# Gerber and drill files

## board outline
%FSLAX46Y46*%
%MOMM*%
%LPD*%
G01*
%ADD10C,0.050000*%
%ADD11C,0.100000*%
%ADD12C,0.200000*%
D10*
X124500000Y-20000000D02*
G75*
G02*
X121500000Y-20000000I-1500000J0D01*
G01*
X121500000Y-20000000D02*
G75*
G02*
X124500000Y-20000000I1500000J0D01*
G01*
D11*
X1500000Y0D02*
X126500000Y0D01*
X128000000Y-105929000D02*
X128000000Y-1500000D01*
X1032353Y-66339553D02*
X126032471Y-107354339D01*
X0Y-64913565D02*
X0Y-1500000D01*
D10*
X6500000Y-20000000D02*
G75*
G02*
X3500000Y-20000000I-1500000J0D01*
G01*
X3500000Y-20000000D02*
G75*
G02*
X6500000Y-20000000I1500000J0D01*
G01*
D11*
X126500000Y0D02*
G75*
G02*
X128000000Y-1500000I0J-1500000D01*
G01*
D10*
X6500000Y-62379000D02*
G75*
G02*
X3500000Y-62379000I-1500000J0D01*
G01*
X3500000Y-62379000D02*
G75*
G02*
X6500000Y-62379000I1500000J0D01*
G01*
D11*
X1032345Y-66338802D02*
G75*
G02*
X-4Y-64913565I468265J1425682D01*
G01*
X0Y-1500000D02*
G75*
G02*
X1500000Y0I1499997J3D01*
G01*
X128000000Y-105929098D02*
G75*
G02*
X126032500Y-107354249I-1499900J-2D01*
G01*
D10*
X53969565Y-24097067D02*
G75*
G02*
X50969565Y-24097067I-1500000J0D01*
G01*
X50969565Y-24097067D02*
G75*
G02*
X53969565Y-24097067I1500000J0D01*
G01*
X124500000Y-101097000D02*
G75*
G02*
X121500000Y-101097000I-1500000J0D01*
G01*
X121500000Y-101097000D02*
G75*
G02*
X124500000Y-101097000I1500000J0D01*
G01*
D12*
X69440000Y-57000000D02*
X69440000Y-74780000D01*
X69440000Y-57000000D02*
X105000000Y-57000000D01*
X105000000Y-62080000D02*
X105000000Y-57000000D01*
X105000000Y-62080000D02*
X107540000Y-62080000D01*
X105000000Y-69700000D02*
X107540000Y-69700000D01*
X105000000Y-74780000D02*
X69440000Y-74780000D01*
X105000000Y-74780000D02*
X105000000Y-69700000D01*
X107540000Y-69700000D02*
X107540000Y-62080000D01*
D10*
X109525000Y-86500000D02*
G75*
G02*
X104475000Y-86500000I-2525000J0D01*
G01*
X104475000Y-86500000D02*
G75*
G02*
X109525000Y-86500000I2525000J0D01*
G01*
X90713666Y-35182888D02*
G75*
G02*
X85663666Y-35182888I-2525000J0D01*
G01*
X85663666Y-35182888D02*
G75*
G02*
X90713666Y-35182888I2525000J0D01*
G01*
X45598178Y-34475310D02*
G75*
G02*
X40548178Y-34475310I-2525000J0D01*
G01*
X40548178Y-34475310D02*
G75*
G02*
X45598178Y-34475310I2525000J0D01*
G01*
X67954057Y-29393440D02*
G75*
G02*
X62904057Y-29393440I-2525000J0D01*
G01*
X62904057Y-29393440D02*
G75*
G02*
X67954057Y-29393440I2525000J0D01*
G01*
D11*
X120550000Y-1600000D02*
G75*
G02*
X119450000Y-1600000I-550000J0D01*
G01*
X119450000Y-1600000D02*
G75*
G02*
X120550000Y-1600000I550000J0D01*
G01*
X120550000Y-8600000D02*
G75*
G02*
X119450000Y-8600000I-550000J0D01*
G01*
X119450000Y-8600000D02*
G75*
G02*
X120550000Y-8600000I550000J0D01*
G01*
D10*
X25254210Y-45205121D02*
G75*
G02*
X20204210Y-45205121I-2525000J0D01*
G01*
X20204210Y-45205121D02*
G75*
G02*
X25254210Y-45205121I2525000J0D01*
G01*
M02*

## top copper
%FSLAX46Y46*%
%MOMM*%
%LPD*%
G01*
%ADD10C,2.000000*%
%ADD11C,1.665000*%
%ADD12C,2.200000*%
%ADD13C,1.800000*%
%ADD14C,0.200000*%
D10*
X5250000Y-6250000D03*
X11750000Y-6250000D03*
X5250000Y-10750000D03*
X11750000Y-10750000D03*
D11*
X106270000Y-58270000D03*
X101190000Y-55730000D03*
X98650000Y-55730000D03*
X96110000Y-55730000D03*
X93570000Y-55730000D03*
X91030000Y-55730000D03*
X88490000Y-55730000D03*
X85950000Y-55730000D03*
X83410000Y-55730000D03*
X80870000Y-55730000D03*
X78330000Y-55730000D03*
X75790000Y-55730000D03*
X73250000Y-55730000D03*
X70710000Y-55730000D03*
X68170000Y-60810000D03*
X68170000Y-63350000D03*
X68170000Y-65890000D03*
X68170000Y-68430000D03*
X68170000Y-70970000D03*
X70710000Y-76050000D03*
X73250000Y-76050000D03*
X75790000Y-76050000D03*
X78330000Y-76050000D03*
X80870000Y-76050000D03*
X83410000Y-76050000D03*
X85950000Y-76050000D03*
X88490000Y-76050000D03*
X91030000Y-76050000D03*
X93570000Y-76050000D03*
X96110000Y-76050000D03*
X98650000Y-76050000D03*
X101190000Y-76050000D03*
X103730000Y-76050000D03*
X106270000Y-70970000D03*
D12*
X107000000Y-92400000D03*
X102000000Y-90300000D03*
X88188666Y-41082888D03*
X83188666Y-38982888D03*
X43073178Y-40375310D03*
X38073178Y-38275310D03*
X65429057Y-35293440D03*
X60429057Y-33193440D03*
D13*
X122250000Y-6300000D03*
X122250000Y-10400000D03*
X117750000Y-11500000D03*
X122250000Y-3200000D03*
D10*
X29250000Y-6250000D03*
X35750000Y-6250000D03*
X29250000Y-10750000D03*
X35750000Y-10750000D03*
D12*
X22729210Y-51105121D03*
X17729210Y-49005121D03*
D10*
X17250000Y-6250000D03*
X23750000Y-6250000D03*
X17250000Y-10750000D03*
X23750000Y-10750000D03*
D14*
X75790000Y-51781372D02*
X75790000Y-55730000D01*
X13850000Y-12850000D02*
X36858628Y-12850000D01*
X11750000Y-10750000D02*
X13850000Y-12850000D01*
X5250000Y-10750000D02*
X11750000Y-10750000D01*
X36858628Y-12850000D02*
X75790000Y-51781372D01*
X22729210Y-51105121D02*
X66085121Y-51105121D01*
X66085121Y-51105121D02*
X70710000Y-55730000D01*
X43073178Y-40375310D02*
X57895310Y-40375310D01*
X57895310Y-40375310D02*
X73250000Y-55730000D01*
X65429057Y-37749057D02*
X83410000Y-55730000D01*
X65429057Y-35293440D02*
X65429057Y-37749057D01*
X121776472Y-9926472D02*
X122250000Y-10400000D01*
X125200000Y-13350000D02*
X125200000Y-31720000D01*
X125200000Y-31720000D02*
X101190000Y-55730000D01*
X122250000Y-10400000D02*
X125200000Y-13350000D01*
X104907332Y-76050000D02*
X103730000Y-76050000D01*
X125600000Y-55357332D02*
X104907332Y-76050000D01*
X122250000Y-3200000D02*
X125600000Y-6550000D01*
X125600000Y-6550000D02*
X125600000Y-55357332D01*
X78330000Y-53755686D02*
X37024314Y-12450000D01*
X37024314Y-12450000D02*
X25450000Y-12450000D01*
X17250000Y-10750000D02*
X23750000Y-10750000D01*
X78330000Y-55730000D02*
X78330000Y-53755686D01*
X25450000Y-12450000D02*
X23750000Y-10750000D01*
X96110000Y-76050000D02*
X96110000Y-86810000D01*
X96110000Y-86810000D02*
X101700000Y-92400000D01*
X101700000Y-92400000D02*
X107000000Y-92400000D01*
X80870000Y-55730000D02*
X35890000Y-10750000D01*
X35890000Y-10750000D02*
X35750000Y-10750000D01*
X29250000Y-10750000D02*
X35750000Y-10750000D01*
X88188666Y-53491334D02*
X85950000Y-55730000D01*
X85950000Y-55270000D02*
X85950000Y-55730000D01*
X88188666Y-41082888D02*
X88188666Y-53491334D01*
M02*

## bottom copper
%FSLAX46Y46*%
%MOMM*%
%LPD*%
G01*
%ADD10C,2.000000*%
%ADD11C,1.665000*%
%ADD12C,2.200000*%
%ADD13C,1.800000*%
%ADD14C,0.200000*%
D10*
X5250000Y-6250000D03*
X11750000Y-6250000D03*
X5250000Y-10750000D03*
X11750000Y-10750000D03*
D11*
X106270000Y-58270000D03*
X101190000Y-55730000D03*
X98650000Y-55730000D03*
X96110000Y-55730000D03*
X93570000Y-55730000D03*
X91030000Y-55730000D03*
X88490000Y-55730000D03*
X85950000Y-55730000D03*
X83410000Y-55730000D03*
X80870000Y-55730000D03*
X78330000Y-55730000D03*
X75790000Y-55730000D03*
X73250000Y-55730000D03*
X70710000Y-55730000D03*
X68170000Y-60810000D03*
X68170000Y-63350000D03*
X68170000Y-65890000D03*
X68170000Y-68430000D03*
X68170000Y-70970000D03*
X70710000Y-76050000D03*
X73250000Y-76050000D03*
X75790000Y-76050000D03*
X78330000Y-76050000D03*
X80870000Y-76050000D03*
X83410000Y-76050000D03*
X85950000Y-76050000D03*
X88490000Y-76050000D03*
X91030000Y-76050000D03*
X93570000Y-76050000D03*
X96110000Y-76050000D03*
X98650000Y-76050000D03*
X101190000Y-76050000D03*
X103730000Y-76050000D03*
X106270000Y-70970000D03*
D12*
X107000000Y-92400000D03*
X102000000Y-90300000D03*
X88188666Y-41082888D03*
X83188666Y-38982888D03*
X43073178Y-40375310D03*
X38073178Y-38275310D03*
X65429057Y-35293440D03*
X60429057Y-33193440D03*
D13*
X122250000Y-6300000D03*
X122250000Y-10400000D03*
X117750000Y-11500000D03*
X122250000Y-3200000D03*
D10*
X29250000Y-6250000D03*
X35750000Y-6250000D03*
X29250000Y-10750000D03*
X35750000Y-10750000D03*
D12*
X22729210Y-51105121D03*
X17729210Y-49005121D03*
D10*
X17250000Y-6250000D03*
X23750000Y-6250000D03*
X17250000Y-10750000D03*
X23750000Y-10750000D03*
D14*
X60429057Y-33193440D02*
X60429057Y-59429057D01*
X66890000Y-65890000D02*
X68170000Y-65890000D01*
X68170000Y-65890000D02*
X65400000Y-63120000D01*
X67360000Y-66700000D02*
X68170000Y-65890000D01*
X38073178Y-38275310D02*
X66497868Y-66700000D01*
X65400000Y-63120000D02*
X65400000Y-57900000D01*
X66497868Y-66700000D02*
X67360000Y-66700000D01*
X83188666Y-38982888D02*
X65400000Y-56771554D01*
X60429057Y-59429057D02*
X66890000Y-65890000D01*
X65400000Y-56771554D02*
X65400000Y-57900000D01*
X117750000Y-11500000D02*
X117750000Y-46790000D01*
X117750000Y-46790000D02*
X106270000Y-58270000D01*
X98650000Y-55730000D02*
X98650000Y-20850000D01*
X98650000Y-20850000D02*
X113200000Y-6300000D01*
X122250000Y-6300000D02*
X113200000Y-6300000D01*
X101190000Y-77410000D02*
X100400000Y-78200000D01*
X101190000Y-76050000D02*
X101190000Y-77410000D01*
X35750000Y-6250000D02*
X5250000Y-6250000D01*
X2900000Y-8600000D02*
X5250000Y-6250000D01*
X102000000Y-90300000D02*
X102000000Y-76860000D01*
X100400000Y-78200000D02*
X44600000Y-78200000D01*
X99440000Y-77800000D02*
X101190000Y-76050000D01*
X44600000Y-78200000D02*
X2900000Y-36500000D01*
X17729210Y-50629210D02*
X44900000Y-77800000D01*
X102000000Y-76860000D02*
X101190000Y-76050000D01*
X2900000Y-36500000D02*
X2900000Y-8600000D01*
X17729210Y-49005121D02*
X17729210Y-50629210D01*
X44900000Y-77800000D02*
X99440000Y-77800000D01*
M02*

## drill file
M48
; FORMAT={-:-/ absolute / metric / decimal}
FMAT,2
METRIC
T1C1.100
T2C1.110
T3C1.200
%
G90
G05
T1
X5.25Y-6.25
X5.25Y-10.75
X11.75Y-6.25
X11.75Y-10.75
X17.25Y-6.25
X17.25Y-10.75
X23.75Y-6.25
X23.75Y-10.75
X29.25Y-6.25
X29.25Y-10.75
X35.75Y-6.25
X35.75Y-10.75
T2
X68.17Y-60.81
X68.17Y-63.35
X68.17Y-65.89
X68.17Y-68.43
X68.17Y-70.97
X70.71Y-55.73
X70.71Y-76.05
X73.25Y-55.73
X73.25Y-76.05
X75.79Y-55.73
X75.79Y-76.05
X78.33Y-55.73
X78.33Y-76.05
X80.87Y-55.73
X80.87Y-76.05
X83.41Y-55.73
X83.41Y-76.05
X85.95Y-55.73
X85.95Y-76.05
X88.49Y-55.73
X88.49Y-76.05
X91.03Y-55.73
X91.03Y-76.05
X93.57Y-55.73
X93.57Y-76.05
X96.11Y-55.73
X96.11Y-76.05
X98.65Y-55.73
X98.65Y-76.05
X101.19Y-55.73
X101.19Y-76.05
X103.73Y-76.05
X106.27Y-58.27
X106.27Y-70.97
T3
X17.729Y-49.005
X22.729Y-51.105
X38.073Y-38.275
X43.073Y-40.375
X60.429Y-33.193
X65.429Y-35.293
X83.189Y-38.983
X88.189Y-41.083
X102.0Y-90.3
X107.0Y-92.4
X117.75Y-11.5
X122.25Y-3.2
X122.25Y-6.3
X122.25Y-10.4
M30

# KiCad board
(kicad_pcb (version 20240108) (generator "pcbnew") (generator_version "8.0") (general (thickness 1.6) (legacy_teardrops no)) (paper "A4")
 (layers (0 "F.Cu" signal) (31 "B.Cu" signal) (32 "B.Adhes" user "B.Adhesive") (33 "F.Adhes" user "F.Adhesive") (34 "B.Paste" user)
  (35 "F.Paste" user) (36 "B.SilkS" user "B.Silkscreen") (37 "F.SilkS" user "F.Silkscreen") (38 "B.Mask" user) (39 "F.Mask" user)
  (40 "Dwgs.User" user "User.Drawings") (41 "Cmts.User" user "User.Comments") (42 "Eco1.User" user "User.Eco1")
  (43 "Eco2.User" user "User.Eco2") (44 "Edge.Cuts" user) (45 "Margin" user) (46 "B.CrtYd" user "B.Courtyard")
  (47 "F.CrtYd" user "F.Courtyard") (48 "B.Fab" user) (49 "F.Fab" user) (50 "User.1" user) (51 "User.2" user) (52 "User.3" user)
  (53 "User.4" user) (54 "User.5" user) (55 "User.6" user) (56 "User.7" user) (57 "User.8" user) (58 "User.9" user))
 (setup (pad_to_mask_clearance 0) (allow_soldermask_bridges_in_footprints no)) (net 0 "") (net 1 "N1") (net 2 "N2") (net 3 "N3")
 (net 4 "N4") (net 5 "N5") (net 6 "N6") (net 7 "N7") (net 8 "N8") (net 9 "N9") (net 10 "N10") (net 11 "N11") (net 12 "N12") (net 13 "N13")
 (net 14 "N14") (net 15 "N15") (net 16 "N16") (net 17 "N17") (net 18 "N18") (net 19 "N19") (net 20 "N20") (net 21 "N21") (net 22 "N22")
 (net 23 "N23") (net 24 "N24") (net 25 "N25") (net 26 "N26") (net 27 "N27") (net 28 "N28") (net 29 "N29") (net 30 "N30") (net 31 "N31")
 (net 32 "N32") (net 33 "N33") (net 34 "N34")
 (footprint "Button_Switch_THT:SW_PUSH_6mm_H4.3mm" (layer "F.Cu") (at 5.25 6.25)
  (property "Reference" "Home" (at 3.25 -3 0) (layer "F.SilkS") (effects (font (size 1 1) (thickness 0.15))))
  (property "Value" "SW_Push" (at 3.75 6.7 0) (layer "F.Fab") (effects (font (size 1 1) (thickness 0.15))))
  (pad "1" thru_hole circle (at 0 0 90) (size 2 2) (drill 1.1) (layers "*.Cu" "*.Mask") (remove_unused_layers no) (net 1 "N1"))
  (pad "1" thru_hole circle (at 6.5 0 90) (size 2 2) (drill 1.1) (layers "*.Cu" "*.Mask") (remove_unused_layers no) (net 1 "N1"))
  (pad "2" thru_hole circle (at 0 4.5 90) (size 2 2) (drill 1.1) (layers "*.Cu" "*.Mask") (remove_unused_layers no) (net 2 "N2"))
  (pad "2" thru_hole circle (at 6.5 4.5 90) (size 2 2) (drill 1.1) (layers "*.Cu" "*.Mask") (remove_unused_layers no) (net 2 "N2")))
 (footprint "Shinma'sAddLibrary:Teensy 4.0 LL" (layer "F.Cu") (at 105 74.78 180)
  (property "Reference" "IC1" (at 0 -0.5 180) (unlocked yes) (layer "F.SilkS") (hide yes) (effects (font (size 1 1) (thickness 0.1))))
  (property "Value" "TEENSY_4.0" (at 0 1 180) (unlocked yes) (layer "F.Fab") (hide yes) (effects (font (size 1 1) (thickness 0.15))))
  (fp_line (start 35.56 17.78) (end 35.56 0) (stroke (width 0.2) (type solid)) (layer "Edge.Cuts"))
  (fp_line (start 35.56 17.78) (end 0 17.78) (stroke (width 0.2) (type solid)) (layer "Edge.Cuts"))
  (fp_line (start 0 12.7) (end 0 17.78) (stroke (width 0.2) (type default)) (layer "Edge.Cuts"))
  (fp_line (start 0 12.7) (end -2.54 12.7) (stroke (width 0.2) (type default)) (layer "Edge.Cuts"))
  (fp_line (start 0 5.08) (end -2.54 5.08) (stroke (width 0.2) (type default)) (layer "Edge.Cuts"))
  (fp_line (start 0 0) (end 35.56 0) (stroke (width 0.2) (type solid)) (layer "Edge.Cuts"))
  (fp_line (start 0 0) (end 0 5.08) (stroke (width 0.2) (type default)) (layer "Edge.Cuts"))
  (fp_line (start -2.54 5.08) (end -2.54 12.7) (stroke (width 0.2) (type default)) (layer "Edge.Cuts"))
  (pad "1" thru_hole circle (at -1.27 16.51 180) (size 1.665 1.665) (drill 1.11) (layers "*.Cu" "*.Mask") (remove_unused_layers no)
   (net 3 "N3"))
  (pad "2" thru_hole circle (at 3.81 19.05 180) (size 1.665 1.665) (drill 1.11) (layers "*.Cu" "*.Mask") (remove_unused_layers no)
   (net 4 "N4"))
  (pad "3" thru_hole circle (at 6.35 19.05 180) (size 1.665 1.665) (drill 1.11) (layers "*.Cu" "*.Mask") (remove_unused_layers no)
   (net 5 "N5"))
  (pad "4" thru_hole circle (at 8.89 19.05 180) (size 1.665 1.665) (drill 1.11) (layers "*.Cu" "*.Mask") (remove_unused_layers no)
   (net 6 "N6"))
  (pad "5" thru_hole circle (at 11.43 19.05 180) (size 1.665 1.665) (drill 1.11) (layers "*.Cu" "*.Mask") (remove_unused_layers no)
   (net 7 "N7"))
  (pad "6" thru_hole circle (at 13.97 19.05 180) (size 1.665 1.665) (drill 1.11) (layers "*.Cu" "*.Mask") (remove_unused_layers no)
   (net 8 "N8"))
  (pad "7" thru_hole circle (at 16.51 19.05 180) (size 1.665 1.665) (drill 1.11) (layers "*.Cu" "*.Mask") (remove_unused_layers no)
   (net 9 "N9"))
  (pad "8" thru_hole circle (at 19.05 19.05 180) (size 1.665 1.665) (drill 1.11) (layers "*.Cu" "*.Mask") (remove_unused_layers no)
   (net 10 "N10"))
  (pad "9" thru_hole circle (at 21.59 19.05 180) (size 1.665 1.665) (drill 1.11) (layers "*.Cu" "*.Mask") (remove_unused_layers no)
   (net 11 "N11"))
  (pad "10" thru_hole circle (at 24.13 19.05 180) (size 1.665 1.665) (drill 1.11) (layers "*.Cu" "*.Mask") (remove_unused_layers no)
   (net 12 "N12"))
  (pad "11" thru_hole circle (at 26.67 19.05 180) (size 1.665 1.665) (drill 1.11) (layers "*.Cu" "*.Mask") (remove_unused_layers no)
   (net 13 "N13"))
  (pad "12" thru_hole circle (at 29.21 19.05 180) (size 1.665 1.665) (drill 1.11) (layers "*.Cu" "*.Mask") (remove_unused_layers no)
   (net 2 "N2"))
  (pad "13" thru_hole circle (at 31.75 19.05 180) (size 1.665 1.665) (drill 1.11) (layers "*.Cu" "*.Mask") (remove_unused_layers no)
   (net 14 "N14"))
  (pad "14" thru_hole circle (at 34.29 19.05 180) (size 1.665 1.665) (drill 1.11) (layers "*.Cu" "*.Mask") (remove_unused_layers no)
   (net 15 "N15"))
  (pad "15" thru_hole circle (at 36.83 13.97 180) (size 1.665 1.665) (drill 1.11) (layers "*.Cu" "*.Mask") (remove_unused_layers no)
   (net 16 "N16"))
  (pad "16" thru_hole circle (at 36.83 11.43 180) (size 1.665 1.665) (drill 1.11) (layers "*.Cu" "*.Mask") (remove_unused_layers no)
   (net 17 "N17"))
  (pad "17" thru_hole circle (at 36.83 8.89 180) (size 1.665 1.665) (drill 1.11) (layers "*.Cu" "*.Mask") (remove_unused_layers no)
   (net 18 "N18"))
  (pad "18" thru_hole circle (at 36.83 6.35 180) (size 1.665 1.665) (drill 1.11) (layers "*.Cu" "*.Mask") (remove_unused_layers no)
   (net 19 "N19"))
  (pad "19" thru_hole circle (at 36.83 3.81 180) (size 1.665 1.665) (drill 1.11) (layers "*.Cu" "*.Mask") (remove_unused_layers no)
   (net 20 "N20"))
  (pad "20" thru_hole circle (at 34.29 -1.27 180) (size 1.665 1.665) (drill 1.11) (layers "*.Cu" "*.Mask") (remove_unused_layers no)
   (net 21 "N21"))
  (pad "21" thru_hole circle (at 31.75 -1.27 180) (size 1.665 1.665) (drill 1.11) (layers "*.Cu" "*.Mask") (remove_unused_layers no)
   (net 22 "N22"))
  (pad "22" thru_hole circle (at 29.21 -1.27 180) (size 1.665 1.665) (drill 1.11) (layers "*.Cu" "*.Mask") (remove_unused_layers no)
   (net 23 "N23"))
  (pad "23" thru_hole circle (at 26.67 -1.27 180) (size 1.665 1.665) (drill 1.11) (layers "*.Cu" "*.Mask") (remove_unused_layers no)
   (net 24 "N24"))
  (pad "24" thru_hole circle (at 24.13 -1.27 180) (size 1.665 1.665) (drill 1.11) (layers "*.Cu" "*.Mask") (remove_unused_layers no)
   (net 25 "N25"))
  (pad "25" thru_hole circle (at 21.59 -1.27 180) (size 1.665 1.665) (drill 1.11) (layers "*.Cu" "*.Mask") (remove_unused_layers no)
   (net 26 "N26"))
  (pad "26" thru_hole circle (at 19.05 -1.27 180) (size 1.665 1.665) (drill 1.11) (layers "*.Cu" "*.Mask") (remove_unused_layers no)
   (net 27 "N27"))
  (pad "27" thru_hole circle (at 16.51 -1.27 180) (size 1.665 1.665) (drill 1.11) (layers "*.Cu" "*.Mask") (remove_unused_layers no)
   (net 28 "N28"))
  (pad "28" thru_hole circle (at 13.97 -1.27 180) (size 1.665 1.665) (drill 1.11) (layers "*.Cu" "*.Mask") (remove_unused_layers no)
   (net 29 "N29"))
  (pad "29" thru_hole circle (at 11.43 -1.27 180) (size 1.665 1.665) (drill 1.11) (layers "*.Cu" "*.Mask") (remove_unused_layers no)
   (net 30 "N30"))
  (pad "30" thru_hole circle (at 8.89 -1.27 180) (size 1.665 1.665) (drill 1.11) (layers "*.Cu" "*.Mask") (remove_unused_layers no)
   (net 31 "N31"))
  (pad "31" thru_hole circle (at 6.35 -1.27 180) (size 1.665 1.665) (drill 1.11) (layers "*.Cu" "*.Mask") (remove_unused_layers no)
   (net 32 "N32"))
  (pad "32" thru_hole circle (at 3.81 -1.27 180) (size 1.665 1.665) (drill 1.11) (layers "*.Cu" "*.Mask") (remove_unused_layers no)
   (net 1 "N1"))
  (pad "33" thru_hole circle (at 1.27 -1.27 180) (size 1.665 1.665) (drill 1.11) (layers "*.Cu" "*.Mask") (remove_unused_layers no)
   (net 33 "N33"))
  (pad "34" thru_hole circle (at -1.27 3.81 180) (size 1.665 1.665) (drill 1.11) (layers "*.Cu" "*.Mask") (remove_unused_layers no)
   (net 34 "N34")))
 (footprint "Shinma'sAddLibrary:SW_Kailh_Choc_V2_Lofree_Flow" (layer "F.Cu") (at 107 86.5)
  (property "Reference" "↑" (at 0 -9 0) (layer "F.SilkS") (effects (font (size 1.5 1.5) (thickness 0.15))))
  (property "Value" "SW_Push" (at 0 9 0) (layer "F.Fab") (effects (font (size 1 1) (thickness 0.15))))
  (fp_circle (center 0 0) (end 2.525 0) (stroke (width 0.05) (type default)) (fill none) (layer "Edge.Cuts"))
  (pad "1" thru_hole circle (at 0 5.9) (size 2.2 2.2) (drill 1.2) (layers "*.Cu" "*.Mask") (remove_unused_layers no) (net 31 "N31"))
  (pad "2" thru_hole circle (at -5 3.8) (size 2.2 2.2) (drill 1.2) (layers "*.Cu" "*.Mask") (remove_unused_layers no) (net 1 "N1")))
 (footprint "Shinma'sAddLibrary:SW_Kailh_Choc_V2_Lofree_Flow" (layer "F.Cu") (at 88.188666 35.182888)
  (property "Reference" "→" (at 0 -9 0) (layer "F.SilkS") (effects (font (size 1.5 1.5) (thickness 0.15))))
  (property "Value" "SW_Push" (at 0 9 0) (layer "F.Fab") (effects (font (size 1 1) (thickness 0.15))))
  (fp_circle (center 0 0) (end 2.525 0) (stroke (width 0.05) (type default)) (fill none) (layer "Edge.Cuts"))
  (pad "1" thru_hole circle (at 0 5.9) (size 2.2 2.2) (drill 1.2) (layers "*.Cu" "*.Mask") (remove_unused_layers no) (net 10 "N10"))
  (pad "2" thru_hole circle (at -5 3.8) (size 2.2 2.2) (drill 1.2) (layers "*.Cu" "*.Mask") (remove_unused_layers no) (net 18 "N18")))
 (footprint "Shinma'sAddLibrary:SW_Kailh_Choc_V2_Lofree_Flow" (layer "F.Cu") (at 43.073178 34.47531)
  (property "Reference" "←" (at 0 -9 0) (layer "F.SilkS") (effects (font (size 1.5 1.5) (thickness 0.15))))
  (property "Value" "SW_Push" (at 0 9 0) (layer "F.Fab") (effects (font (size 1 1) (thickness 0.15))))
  (fp_circle (center 0 0) (end 2.525 0) (stroke (width 0.05) (type default)) (fill none) (layer "Edge.Cuts"))
  (pad "1" thru_hole circle (at 0 5.9) (size 2.2 2.2) (drill 1.2) (layers "*.Cu" "*.Mask") (remove_unused_layers no) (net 14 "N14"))
  (pad "2" thru_hole circle (at -5 3.8) (size 2.2 2.2) (drill 1.2) (layers "*.Cu" "*.Mask") (remove_unused_layers no) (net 18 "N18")))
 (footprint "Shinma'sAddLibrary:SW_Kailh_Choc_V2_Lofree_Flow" (layer "F.Cu") (at 65.429057 29.39344)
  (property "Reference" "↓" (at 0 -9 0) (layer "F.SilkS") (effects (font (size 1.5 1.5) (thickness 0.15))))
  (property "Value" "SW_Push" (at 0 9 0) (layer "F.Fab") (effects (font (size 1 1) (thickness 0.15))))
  (fp_circle (center 0 0) (end 2.525 0) (stroke (width 0.05) (type default)) (fill none) (layer "Edge.Cuts"))
  (pad "1" thru_hole circle (at 0 5.9) (size 2.2 2.2) (drill 1.2) (layers "*.Cu" "*.Mask") (remove_unused_layers no) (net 11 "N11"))
  (pad "2" thru_hole circle (at -5 3.8) (size 2.2 2.2) (drill 1.2) (layers "*.Cu" "*.Mask") (remove_unused_layers no) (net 18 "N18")))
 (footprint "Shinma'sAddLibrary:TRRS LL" (layer "F.Cu") (at 117 12 90)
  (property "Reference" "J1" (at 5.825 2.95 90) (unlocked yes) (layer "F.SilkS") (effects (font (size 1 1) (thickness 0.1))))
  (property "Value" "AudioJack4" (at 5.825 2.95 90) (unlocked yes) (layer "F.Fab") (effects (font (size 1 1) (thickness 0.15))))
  (fp_circle (center 10.4 3) (end 10.95 3) (stroke (width 0.1) (type default)) (fill none) (layer "Edge.Cuts"))
  (fp_circle (center 3.4 3) (end 3.95 3) (stroke (width 0.1) (type default)) (fill none) (layer "Edge.Cuts"))
  (pad "R1" thru_hole circle (at 5.7 5.25 90) (size 1.8 1.8) (drill 1.2) (layers "*.Cu" "*.Mask") (remove_unused_layers no) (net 5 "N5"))
  (pad "R2" thru_hole circle (at 1.6 5.25 90) (size 1.8 1.8) (drill 1.2) (layers "*.Cu" "*.Mask") (remove_unused_layers no) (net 4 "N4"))
  (pad "S" thru_hole circle (at 0.5 0.75 90) (size 1.8 1.8) (drill 1.2) (layers "*.Cu" "*.Mask") (remove_unused_layers no) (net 3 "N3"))
  (pad "T" thru_hole circle (at 8.8 5.25 90) (size 1.8 1.8) (drill 1.2) (layers "*.Cu" "*.Mask") (remove_unused_layers no) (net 33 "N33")))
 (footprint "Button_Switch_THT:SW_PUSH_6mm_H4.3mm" (layer "F.Cu") (at 29.25 6.25)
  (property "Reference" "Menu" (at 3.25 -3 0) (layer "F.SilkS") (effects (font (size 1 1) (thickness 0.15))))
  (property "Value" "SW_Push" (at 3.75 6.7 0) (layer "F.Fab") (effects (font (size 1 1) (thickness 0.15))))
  (pad "1" thru_hole circle (at 0 0 90) (size 2 2) (drill 1.1) (layers "*.Cu" "*.Mask") (remove_unused_layers no) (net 1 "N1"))
  (pad "1" thru_hole circle (at 6.5 0 90) (size 2 2) (drill 1.1) (layers "*.Cu" "*.Mask") (remove_unused_layers no) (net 1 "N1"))
  (pad "2" thru_hole circle (at 0 4.5 90) (size 2 2) (drill 1.1) (layers "*.Cu" "*.Mask") (remove_unused_layers no) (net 12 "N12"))
  (pad "2" thru_hole circle (at 6.5 4.5 90) (size 2 2) (drill 1.1) (layers "*.Cu" "*.Mask") (remove_unused_layers no) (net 12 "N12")))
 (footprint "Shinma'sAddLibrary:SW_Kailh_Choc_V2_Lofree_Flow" (layer "F.Cu") (at 22.72921 45.205121)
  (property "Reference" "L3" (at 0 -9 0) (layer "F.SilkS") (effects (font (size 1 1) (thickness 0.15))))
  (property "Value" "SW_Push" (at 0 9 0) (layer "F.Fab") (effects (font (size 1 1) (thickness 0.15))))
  (fp_circle (center 0 0) (end 2.525 0) (stroke (width 0.05) (type default)) (fill none) (layer "Edge.Cuts"))
  (pad "1" thru_hole circle (at 0 5.9) (size 2.2 2.2) (drill 1.2) (layers "*.Cu" "*.Mask") (remove_unused_layers no) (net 15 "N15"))
  (pad "2" thru_hole circle (at -5 3.8) (size 2.2 2.2) (drill 1.2) (layers "*.Cu" "*.Mask") (remove_unused_layers no) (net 1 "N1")))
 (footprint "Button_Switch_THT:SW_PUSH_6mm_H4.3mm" (layer "F.Cu") (at 17.25 6.25)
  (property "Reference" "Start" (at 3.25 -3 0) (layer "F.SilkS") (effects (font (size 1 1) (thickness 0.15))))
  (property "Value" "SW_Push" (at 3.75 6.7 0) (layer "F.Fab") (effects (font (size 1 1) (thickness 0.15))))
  (pad "1" thru_hole circle (at 0 0 90) (size 2 2) (drill 1.1) (layers "*.Cu" "*.Mask") (remove_unused_layers no) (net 1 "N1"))
  (pad "1" thru_hole circle (at 6.5 0 90) (size 2 2) (drill 1.1) (layers "*.Cu" "*.Mask") (remove_unused_layers no) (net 1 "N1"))
  (pad "2" thru_hole circle (at 0 4.5 90) (size 2 2) (drill 1.1) (layers "*.Cu" "*.Mask") (remove_unused_layers no) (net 13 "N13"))
  (pad "2" thru_hole circle (at 6.5 4.5 90) (size 2 2) (drill 1.1) (layers "*.Cu" "*.Mask") (remove_unused_layers no) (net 13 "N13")))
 (gr_circle (center 123 20) (end 124.5 20) (stroke (width 0.05) (type default)) (fill none) (layer "Edge.Cuts"))
 (gr_line (start 1.5 0) (end 126.5 0) (stroke (width 0.1) (type default)) (layer "Edge.Cuts"))
 (gr_line (start 128 105.929) (end 128 1.5) (stroke (width 0.1) (type default)) (layer "Edge.Cuts"))
 (gr_line (start 1.032353 66.339553) (end 126.032471 107.354339) (stroke (width 0.1) (type default)) (layer "Edge.Cuts"))
 (gr_line (start 0 64.913565) (end 0 1.5) (stroke (width 0.1) (type default)) (layer "Edge.Cuts"))
 (gr_circle (center 5 20) (end 6.5 20) (stroke (width 0.05) (type default)) (fill none) (layer "Edge.Cuts"))
 (gr_arc (start 126.5 0) (mid 127.56066 0.43934) (end 128 1.5) (stroke (width 0.1) (type default)) (layer "Edge.Cuts"))
 (gr_circle (center 5 62.379) (end 6.5 62.379) (stroke (width 0.05) (type default)) (fill none) (layer "Edge.Cuts"))
 (gr_arc (start 1.032345 66.338802) (mid 0.285315 65.793401) (end 0 64.913565) (stroke (width 0.1) (type default)) (layer "Edge.Cuts"))
 (gr_arc (start 0 1.5) (mid 0.439339 0.439339) (end 1.5 0) (stroke (width 0.1) (type default)) (layer "Edge.Cuts"))
 (gr_arc (start 128 105.929098) (mid 127.379985 107.14387) (end 126.032471 107.354339) (stroke (width 0.1) (type default))
  (layer "Edge.Cuts"))
 (gr_circle (center 52.469565 24.097067) (end 53.969565 24.097067) (stroke (width 0.05) (type default)) (fill none) (layer "Edge.Cuts"))
 (gr_circle (center 123 101.097) (end 124.5 101.097) (stroke (width 0.05) (type default)) (fill none) (layer "Edge.Cuts"))
 (segment (start 75.79 51.781372) (end 75.79 55.73) (width 0.2) (layer "F.Cu") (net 2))
 (segment (start 13.85 12.85) (end 36.858628 12.85) (width 0.2) (layer "F.Cu") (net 2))
 (segment (start 11.75 10.75) (end 13.85 12.85) (width 0.2) (layer "F.Cu") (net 2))
 (segment (start 5.25 10.75) (end 11.75 10.75) (width 0.2) (layer "F.Cu") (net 2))
 (segment (start 36.858628 12.85) (end 75.79 51.781372) (width 0.2) (layer "F.Cu") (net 2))
 (segment (start 22.72921 51.105121) (end 66.085121 51.105121) (width 0.2) (layer "F.Cu") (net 15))
 (segment (start 66.085121 51.105121) (end 70.71 55.73) (width 0.2) (layer "F.Cu") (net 15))
 (segment (start 60.429057 33.19344) (end 60.429057 59.429057) (width 0.2) (layer "B.Cu") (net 18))
 (segment (start 66.89 65.89) (end 68.17 65.89) (width 0.2) (layer "B.Cu") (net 18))
 (segment (start 68.17 65.89) (end 65.4 63.12) (width 0.2) (layer "B.Cu") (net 18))
 (segment (start 67.36 66.7) (end 68.17 65.89) (width 0.2) (layer "B.Cu") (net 18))
 (segment (start 38.073178 38.27531) (end 66.497868 66.7) (width 0.2) (layer "B.Cu") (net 18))
 (segment (start 65.4 63.12) (end 65.4 57.9) (width 0.2) (layer "B.Cu") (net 18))
 (segment (start 66.497868 66.7) (end 67.36 66.7) (width 0.2) (layer "B.Cu") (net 18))
 (segment (start 83.188666 38.982888) (end 65.4 56.771554) (width 0.2) (layer "B.Cu") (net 18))
 (segment (start 60.429057 59.429057) (end 66.89 65.89) (width 0.2) (layer "B.Cu") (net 18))
 (segment (start 65.4 56.771554) (end 65.4 57.9) (width 0.2) (layer "B.Cu") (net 18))
 (segment (start 43.073178 40.37531) (end 57.89531 40.37531) (width 0.2) (layer "F.Cu") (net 14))
 (segment (start 57.89531 40.37531) (end 73.25 55.73) (width 0.2) (layer "F.Cu") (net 14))
 (segment (start 117.75 11.5) (end 117.75 46.79) (width 0.2) (layer "B.Cu") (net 3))
 (segment (start 117.75 46.79) (end 106.27 58.27) (width 0.2) (layer "B.Cu") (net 3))
 (segment (start 65.429057 37.749057) (end 83.41 55.73) (width 0.2) (layer "F.Cu") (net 11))
 (segment (start 65.429057 35.29344) (end 65.429057 37.749057) (width 0.2) (layer "F.Cu") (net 11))
 (segment (start 121.776472 9.926472) (end 122.25 10.4) (width 0.2) (layer "F.Cu") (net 4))
 (segment (start 125.2 13.35) (end 125.2 31.72) (width 0.2) (layer "F.Cu") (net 4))
 (segment (start 125.2 31.72) (end 101.19 55.73) (width 0.2) (layer "F.Cu") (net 4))
 (segment (start 122.25 10.4) (end 125.2 13.35) (width 0.2) (layer "F.Cu") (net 4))
 (segment (start 104.907332 76.05) (end 103.73 76.05) (width 0.2) (layer "F.Cu") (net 33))
 (segment (start 125.6 55.357332) (end 104.907332 76.05) (width 0.2) (layer "F.Cu") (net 33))
 (segment (start 122.25 3.2) (end 125.6 6.55) (width 0.2) (layer "F.Cu") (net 33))
 (segment (start 125.6 6.55) (end 125.6 55.357332) (width 0.2) (layer "F.Cu") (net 33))
 (segment (start 78.33 53.755686) (end 37.024314 12.45) (width 0.2) (layer "F.Cu") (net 13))
 (segment (start 37.024314 12.45) (end 25.45 12.45) (width 0.2) (layer "F.Cu") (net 13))
 (segment (start 17.25 10.75) (end 23.75 10.75) (width 0.2) (layer "F.Cu") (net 13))
 (segment (start 78.33 55.73) (end 78.33 53.755686) (width 0.2) (layer "F.Cu") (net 13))
 (segment (start 25.45 12.45) (end 23.75 10.75) (width 0.2) (layer "F.Cu") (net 13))
 (segment (start 98.65 55.73) (end 98.65 20.85) (width 0.2) (layer "B.Cu") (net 5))
 (segment (start 98.65 20.85) (end 113.2 6.3) (width 0.2) (layer "B.Cu") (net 5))
 (segment (start 122.25 6.3) (end 113.2 6.3) (width 0.2) (layer "B.Cu") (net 5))
 (segment (start 96.11 76.05) (end 96.11 86.81) (width 0.2) (layer "F.Cu") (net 31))
 (segment (start 96.11 86.81) (end 101.7 92.4) (width 0.2) (layer "F.Cu") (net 31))
 (segment (start 101.7 92.4) (end 107 92.4) (width 0.2) (layer "F.Cu") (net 31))
 (segment (start 101.19 77.41) (end 100.4 78.2) (width 0.2) (layer "B.Cu") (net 1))
 (segment (start 101.19 76.05) (end 101.19 77.41) (width 0.2) (layer "B.Cu") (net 1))
 (segment (start 35.75 6.25) (end 5.25 6.25) (width 0.2) (layer "B.Cu") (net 1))
 (segment (start 2.9 8.6) (end 5.25 6.25) (width 0.2) (layer "B.Cu") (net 1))
 (segment (start 102 90.3) (end 102 76.86) (width 0.2) (layer "B.Cu") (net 1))
 (segment (start 100.4 78.2) (end 44.6 78.2) (width 0.2) (layer "B.Cu") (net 1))
 (segment (start 99.44 77.8) (end 101.19 76.05) (width 0.2) (layer "B.Cu") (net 1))
 (segment (start 44.6 78.2) (end 2.9 36.5) (width 0.2) (layer "B.Cu") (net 1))
 (segment (start 17.72921 50.62921) (end 44.9 77.8) (width 0.2) (layer "B.Cu") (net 1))
 (segment (start 102 76.86) (end 101.19 76.05) (width 0.2) (layer "B.Cu") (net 1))
 (segment (start 2.9 36.5) (end 2.9 8.6) (width 0.2) (layer "B.Cu") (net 1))
 (segment (start 17.72921 49.005121) (end 17.72921 50.62921) (width 0.2) (layer "B.Cu") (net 1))
 (segment (start 44.9 77.8) (end 99.44 77.8) (width 0.2) (layer "B.Cu") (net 1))
 (segment (start 80.87 55.73) (end 35.89 10.75) (width 0.2) (layer "F.Cu") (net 12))
 (segment (start 35.89 10.75) (end 35.75 10.75) (width 0.2) (layer "F.Cu") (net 12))
 (segment (start 29.25 10.75) (end 35.75 10.75) (width 0.2) (layer "F.Cu") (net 12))
 (segment (start 88.188666 53.491334) (end 85.95 55.73) (width 0.2) (layer "F.Cu") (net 10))
 (segment (start 85.95 55.27) (end 85.95 55.73) (width 0.2) (layer "F.Cu") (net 10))
 (segment (start 88.188666 41.082888) (end 88.188666 53.491334) (width 0.2) (layer "F.Cu") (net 10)))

